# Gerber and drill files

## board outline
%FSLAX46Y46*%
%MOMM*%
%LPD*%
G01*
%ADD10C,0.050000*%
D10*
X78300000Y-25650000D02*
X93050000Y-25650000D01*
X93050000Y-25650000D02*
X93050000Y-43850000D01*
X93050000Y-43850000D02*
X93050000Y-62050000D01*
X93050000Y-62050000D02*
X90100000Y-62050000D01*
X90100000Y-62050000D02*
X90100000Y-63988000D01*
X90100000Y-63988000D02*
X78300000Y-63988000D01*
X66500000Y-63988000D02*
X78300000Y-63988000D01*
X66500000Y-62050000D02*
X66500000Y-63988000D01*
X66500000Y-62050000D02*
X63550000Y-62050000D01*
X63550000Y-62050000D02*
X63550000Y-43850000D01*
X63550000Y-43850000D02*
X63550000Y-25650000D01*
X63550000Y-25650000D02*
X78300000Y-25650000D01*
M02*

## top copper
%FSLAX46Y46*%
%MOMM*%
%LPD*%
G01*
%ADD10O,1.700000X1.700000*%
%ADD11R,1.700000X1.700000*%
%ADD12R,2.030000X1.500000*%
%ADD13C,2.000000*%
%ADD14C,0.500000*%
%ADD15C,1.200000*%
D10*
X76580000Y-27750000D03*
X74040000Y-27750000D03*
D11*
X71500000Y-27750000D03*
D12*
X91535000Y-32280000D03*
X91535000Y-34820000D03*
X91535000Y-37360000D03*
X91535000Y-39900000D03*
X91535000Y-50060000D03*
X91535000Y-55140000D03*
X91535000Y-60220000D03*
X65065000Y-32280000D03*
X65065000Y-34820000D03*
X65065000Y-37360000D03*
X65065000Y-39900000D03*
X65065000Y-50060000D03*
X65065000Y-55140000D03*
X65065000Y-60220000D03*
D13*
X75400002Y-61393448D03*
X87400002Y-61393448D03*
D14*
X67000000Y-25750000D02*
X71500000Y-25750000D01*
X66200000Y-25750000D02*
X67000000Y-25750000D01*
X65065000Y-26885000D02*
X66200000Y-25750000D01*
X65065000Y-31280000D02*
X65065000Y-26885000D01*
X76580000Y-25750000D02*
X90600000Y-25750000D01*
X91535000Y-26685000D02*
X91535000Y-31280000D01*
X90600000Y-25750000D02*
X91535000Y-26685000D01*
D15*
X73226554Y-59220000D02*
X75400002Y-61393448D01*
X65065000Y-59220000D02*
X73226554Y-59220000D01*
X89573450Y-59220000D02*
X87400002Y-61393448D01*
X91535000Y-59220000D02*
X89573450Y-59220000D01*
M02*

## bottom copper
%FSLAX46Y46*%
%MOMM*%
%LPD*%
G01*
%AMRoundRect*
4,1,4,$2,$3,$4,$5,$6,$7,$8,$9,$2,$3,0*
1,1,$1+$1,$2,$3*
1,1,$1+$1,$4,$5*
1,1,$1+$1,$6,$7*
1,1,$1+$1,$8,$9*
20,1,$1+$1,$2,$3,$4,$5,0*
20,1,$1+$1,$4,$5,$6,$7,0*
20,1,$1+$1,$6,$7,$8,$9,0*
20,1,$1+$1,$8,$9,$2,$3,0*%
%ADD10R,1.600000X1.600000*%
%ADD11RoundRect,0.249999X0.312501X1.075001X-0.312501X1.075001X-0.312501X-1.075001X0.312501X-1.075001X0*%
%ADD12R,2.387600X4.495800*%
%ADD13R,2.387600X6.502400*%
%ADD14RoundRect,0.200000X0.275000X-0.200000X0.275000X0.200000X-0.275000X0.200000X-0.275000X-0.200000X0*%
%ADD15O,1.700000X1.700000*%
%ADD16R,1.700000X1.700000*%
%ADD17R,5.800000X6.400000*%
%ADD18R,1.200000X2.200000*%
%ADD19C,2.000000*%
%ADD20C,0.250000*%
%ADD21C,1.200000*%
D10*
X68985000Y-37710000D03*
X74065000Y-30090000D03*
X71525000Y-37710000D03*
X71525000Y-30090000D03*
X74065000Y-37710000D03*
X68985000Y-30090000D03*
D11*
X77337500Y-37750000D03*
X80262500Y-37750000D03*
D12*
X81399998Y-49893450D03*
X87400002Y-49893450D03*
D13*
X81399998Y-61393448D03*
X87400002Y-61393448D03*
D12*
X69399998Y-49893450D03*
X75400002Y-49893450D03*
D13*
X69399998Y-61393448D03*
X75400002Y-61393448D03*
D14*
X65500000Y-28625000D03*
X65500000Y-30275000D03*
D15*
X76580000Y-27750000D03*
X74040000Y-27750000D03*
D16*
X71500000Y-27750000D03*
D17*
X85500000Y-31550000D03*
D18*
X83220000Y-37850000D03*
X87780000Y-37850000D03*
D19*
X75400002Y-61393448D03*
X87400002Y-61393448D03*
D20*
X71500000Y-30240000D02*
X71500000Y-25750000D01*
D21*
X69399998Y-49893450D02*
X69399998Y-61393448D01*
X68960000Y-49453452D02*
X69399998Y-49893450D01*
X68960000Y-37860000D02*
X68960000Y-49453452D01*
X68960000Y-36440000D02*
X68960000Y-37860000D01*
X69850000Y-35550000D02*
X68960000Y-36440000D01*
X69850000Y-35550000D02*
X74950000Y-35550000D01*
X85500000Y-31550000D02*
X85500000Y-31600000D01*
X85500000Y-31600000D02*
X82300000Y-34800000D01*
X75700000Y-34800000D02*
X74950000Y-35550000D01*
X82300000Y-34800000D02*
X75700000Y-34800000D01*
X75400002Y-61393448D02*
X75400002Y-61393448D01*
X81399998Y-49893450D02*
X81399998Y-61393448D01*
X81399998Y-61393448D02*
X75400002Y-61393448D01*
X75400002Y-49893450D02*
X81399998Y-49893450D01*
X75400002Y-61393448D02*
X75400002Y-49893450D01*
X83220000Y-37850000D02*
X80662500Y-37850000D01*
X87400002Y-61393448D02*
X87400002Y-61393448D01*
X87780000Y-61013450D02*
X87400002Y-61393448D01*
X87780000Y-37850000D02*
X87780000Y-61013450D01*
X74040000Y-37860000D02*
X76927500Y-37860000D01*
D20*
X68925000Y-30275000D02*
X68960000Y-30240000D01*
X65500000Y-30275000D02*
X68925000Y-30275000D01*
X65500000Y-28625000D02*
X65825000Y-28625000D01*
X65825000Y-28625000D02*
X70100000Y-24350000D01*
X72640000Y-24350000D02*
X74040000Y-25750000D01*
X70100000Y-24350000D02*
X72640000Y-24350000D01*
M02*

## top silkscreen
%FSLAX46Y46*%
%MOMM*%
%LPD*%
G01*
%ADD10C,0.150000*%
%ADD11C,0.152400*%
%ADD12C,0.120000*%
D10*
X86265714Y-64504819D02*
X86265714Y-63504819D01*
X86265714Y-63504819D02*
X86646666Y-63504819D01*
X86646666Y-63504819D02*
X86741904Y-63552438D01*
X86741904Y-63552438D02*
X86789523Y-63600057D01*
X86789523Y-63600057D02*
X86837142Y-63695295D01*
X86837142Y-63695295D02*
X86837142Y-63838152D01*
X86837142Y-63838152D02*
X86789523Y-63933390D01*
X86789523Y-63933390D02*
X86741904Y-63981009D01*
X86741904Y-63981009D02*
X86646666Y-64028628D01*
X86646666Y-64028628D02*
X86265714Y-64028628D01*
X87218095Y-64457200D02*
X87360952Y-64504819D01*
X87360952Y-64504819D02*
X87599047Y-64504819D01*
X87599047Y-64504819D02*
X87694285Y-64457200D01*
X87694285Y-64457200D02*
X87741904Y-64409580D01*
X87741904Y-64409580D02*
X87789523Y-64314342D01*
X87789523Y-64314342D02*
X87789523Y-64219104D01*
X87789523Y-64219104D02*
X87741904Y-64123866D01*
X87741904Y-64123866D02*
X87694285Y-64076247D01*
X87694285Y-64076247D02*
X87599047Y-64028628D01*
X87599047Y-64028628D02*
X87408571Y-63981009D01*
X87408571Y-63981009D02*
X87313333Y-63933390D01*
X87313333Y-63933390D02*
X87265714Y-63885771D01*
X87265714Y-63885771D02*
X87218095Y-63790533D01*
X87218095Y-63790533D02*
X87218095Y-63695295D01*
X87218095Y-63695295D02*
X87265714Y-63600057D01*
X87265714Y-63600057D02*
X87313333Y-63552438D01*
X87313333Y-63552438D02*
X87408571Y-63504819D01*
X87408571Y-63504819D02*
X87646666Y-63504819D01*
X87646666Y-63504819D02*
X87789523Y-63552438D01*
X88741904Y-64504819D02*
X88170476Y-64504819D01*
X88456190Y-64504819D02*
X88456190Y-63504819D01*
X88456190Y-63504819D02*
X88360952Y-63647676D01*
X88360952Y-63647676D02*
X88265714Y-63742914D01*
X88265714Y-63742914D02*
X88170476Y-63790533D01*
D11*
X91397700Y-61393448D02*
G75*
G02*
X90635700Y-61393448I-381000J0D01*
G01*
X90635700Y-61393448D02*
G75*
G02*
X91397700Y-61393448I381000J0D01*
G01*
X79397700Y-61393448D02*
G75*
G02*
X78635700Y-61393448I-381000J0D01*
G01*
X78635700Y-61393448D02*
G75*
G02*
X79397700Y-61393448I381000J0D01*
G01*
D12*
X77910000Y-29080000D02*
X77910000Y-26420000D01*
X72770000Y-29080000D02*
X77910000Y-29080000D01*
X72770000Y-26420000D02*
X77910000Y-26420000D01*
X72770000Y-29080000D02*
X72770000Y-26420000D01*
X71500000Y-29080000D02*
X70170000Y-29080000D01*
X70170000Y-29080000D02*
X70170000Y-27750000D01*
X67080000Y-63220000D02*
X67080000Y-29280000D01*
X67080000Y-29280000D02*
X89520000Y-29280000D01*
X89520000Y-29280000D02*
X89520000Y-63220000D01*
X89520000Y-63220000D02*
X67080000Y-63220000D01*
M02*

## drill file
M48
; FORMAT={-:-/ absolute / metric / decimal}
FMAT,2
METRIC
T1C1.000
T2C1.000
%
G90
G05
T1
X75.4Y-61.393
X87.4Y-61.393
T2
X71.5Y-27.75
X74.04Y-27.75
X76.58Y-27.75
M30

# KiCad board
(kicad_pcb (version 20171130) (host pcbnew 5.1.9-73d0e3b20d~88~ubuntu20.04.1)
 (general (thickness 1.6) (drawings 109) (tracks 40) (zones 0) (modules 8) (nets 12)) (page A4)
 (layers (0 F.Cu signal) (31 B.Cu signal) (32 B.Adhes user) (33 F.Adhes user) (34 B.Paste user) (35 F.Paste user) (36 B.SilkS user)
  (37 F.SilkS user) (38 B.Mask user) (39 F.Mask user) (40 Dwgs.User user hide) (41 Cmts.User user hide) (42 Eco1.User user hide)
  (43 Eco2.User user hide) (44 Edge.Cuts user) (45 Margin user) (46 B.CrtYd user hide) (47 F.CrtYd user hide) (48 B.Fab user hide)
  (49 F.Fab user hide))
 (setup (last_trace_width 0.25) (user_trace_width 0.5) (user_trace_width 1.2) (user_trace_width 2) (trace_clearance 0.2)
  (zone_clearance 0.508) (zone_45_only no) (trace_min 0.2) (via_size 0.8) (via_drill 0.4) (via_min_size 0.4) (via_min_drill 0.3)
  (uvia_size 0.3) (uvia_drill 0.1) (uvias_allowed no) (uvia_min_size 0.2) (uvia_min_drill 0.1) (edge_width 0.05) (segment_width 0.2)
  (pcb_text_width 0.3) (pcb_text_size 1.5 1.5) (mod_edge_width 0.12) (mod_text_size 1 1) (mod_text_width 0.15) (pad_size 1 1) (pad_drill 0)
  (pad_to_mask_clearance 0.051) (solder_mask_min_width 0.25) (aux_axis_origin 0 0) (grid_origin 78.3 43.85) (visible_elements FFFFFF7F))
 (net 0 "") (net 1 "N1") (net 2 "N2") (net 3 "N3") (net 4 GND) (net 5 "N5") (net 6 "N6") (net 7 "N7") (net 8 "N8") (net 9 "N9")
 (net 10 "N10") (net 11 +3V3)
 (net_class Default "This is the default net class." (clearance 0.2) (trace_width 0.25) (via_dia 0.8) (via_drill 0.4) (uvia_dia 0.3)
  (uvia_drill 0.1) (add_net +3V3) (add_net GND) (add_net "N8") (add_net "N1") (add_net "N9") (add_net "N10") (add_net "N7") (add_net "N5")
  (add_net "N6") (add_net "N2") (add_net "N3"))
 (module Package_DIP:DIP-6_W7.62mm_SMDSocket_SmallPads (layer B.Cu) (at 71.525 33.9 270)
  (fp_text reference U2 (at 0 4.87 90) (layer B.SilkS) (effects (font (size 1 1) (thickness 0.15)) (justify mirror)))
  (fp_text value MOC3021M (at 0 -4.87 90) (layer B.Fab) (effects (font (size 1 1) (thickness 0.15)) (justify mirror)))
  (pad 6 smd rect (at 3.81 2.54 270) (size 1.6 1.6) (layers B.Cu B.Paste B.Mask) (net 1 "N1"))
  (pad 3 smd rect (at -3.81 -2.54 270) (size 1.6 1.6) (layers B.Cu B.Paste B.Mask) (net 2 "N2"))
  (pad 5 smd rect (at 3.81 0 270) (size 1.6 1.6) (layers B.Cu B.Paste B.Mask) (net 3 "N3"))
  (pad 2 smd rect (at -3.81 0 270) (size 1.6 1.6) (layers B.Cu B.Paste B.Mask) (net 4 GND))
  (pad 4 smd rect (at 3.81 -2.54 270) (size 1.6 1.6) (layers B.Cu B.Paste B.Mask) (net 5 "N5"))
  (pad 1 smd rect (at -3.81 2.54 270) (size 1.6 1.6) (layers B.Cu B.Paste B.Mask) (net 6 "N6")))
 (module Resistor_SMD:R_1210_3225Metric (layer B.Cu) (at 78.8 37.75 180)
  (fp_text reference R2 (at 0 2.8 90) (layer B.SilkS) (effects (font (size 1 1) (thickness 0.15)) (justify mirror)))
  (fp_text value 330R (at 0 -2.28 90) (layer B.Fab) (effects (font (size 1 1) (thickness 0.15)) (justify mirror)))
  (pad 2 smd roundrect (at 1.4625 0 180) (size 1.125 2.65) (layers B.Cu B.Paste B.Mask) (roundrect_rratio 0.2222213333333333) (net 5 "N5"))
  (pad 1 smd roundrect (at -1.4625 0 180) (size 1.125 2.65) (layers B.Cu B.Paste B.Mask) (roundrect_rratio 0.2222213333333333) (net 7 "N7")))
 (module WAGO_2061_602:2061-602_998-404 (layer B.Cu) (at 84.4 56.65 180)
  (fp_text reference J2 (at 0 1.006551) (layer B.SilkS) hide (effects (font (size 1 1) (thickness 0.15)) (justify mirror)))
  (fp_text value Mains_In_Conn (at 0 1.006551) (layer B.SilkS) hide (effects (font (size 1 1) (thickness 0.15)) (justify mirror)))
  (fp_circle (center -6.6167 -4.743448) (end -6.2357 -4.743448) (layer F.SilkS) (width 0.1524))
  (pad 2 smd rect (at 3.000002 6.75655 180) (size 2.3876 4.4958) (layers B.Cu B.Paste B.Mask) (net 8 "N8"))
  (pad 1 smd rect (at -3.000002 6.75655 180) (size 2.3876 4.4958) (layers B.Cu B.Paste B.Mask) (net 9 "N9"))
  (pad 2 smd rect (at 3.000002 -4.743448 180) (size 2.3876 6.5024) (layers B.Cu B.Paste B.Mask) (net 8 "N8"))
  (pad 1 smd rect (at -3.000002 -4.743448 180) (size 2.3876 6.5024) (layers B.Cu B.Paste B.Mask) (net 9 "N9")))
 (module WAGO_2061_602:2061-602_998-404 (layer B.Cu) (at 72.4 56.65 180)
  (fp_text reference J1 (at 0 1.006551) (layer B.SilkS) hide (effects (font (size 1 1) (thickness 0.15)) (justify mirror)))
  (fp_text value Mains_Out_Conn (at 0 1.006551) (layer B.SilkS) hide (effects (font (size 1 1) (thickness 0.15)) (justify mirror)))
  (fp_circle (center -6.6167 -4.743448) (end -6.2357 -4.743448) (layer F.SilkS) (width 0.1524))
  (pad 2 smd rect (at 3.000002 6.75655 180) (size 2.3876 4.4958) (layers B.Cu B.Paste B.Mask) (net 1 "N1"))
  (pad 1 smd rect (at -3.000002 6.75655 180) (size 2.3876 4.4958) (layers B.Cu B.Paste B.Mask) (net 8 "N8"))
  (pad 2 smd rect (at 3.000002 -4.743448 180) (size 2.3876 6.5024) (layers B.Cu B.Paste B.Mask) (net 1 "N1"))
  (pad 1 smd rect (at -3.000002 -4.743448 180) (size 2.3876 6.5024) (layers B.Cu B.Paste B.Mask) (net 8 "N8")))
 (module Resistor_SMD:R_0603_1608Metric (layer B.Cu) (at 65.5 29.45 90)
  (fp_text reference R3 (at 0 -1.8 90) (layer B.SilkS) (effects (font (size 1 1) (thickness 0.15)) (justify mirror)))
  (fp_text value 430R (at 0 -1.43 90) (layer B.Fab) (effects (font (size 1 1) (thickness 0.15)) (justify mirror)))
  (pad 2 smd roundrect (at 0.825 0 90) (size 0.8 0.95) (layers B.Cu B.Paste B.Mask) (roundrect_rratio 0.25) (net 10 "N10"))
  (pad 1 smd roundrect (at -0.825 0 90) (size 0.8 0.95) (layers B.Cu B.Paste B.Mask) (roundrect_rratio 0.25) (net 6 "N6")))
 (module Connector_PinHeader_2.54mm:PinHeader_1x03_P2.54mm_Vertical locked (layer F.Cu) (at 71.500 27.750 90.000)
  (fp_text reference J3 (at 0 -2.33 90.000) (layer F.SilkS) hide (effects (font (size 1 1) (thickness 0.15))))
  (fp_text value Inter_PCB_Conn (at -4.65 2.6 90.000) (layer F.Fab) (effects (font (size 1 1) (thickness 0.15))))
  (fp_line (start -1.33 6.41) (end 1.33 6.41) (layer F.SilkS) (width 0.12))
  (fp_line (start -1.33 1.27) (end -1.33 6.41) (layer F.SilkS) (width 0.12))
  (fp_line (start 1.33 1.27) (end 1.33 6.41) (layer F.SilkS) (width 0.12))
  (fp_line (start -1.33 1.27) (end 1.33 1.27) (layer F.SilkS) (width 0.12))
  (fp_line (start -1.33 0) (end -1.33 -1.33) (layer F.SilkS) (width 0.12))
  (fp_line (start -1.33 -1.33) (end 0 -1.33) (layer F.SilkS) (width 0.12))
  (pad 3 thru_hole oval (at 0 5.08 90.000) (size 1.7 1.7) (drill 1) (layers *.Cu *.Mask) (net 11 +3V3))
  (pad 2 thru_hole oval (at 0 2.54 90.000) (size 1.7 1.7) (drill 1) (layers *.Cu *.Mask) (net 10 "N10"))
  (pad 1 thru_hole rect (at 0 0 90.000) (size 1.7 1.7) (drill 1) (layers *.Cu *.Mask) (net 4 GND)))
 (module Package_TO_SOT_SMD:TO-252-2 (layer B.Cu) (at 85.5 33.65 90)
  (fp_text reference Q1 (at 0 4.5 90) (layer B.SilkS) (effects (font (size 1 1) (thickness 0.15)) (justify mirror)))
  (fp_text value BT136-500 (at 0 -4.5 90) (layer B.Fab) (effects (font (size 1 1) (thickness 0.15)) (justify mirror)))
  (pad "" smd rect (at 0.425 -1.525 90) (size 3.05 2.75) (layers B.Paste))
  (pad "" smd rect (at 3.775 1.525 90) (size 3.05 2.75) (layers B.Paste))
  (pad "" smd rect (at 0.425 1.525 90) (size 3.05 2.75) (layers B.Paste))
  (pad "" smd rect (at 3.775 -1.525 90) (size 3.05 2.75) (layers B.Paste))
  (pad 2 smd rect (at 2.1 0 90) (size 6.4 5.8) (layers B.Cu B.Mask) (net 1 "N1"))
  (pad 3 smd rect (at -4.2 -2.28 90) (size 2.2 1.2) (layers B.Cu B.Paste B.Mask) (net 7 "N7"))
  (pad 1 smd rect (at -4.2 2.28 90) (size 2.2 1.2) (layers B.Cu B.Paste B.Mask) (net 9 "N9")))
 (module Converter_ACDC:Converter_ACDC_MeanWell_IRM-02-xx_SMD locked (layer F.Cu) (at 78.300 46.250 180.000)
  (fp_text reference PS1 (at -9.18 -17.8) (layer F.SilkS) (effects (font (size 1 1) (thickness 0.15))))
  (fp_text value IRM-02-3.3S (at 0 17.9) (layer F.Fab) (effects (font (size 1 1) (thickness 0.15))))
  (fp_line (start 11.22 -16.97) (end 11.22 16.97) (layer F.SilkS) (width 0.12))
  (fp_line (start 11.22 16.97) (end -11.22 16.97) (layer F.SilkS) (width 0.12))
  (fp_line (start -11.22 16.97) (end -11.22 -16.97) (layer F.SilkS) (width 0.12))
  (fp_line (start -11.22 -16.97) (end 11.22 -16.97) (layer F.SilkS) (width 0.12))
  (pad 12 smd rect (at -13.235 13.97 90.000) (size 1.5 2.03) (layers F.Cu F.Paste F.Mask) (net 11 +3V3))
  (pad 11 smd rect (at -13.235 11.43 90.000) (size 1.5 2.03) (layers F.Cu F.Paste F.Mask))
  (pad 10 smd rect (at -13.235 8.89 90.000) (size 1.5 2.03) (layers F.Cu F.Paste F.Mask))
  (pad 9 smd rect (at -13.235 6.35 90.000) (size 1.5 2.03) (layers F.Cu F.Paste F.Mask))
  (pad 5 smd rect (at -13.235 -3.81 90.000) (size 1.5 2.03) (layers F.Cu F.Paste F.Mask))
  (pad 3 smd rect (at -13.235 -8.89 90.000) (size 1.5 2.03) (layers F.Cu F.Paste F.Mask))
  (pad 1 smd rect (at -13.235 -13.97 90.000) (size 1.5 2.03) (layers F.Cu F.Paste F.Mask) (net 9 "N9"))
  (pad 13 smd rect (at 13.235 13.97 90.000) (size 1.5 2.03) (layers F.Cu F.Paste F.Mask) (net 4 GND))
  (pad 14 smd rect (at 13.235 11.43 90.000) (size 1.5 2.03) (layers F.Cu F.Paste F.Mask))
  (pad 15 smd rect (at 13.235 8.89 90.000) (size 1.5 2.03) (layers F.Cu F.Paste F.Mask))
  (pad 16 smd rect (at 13.235 6.35 90.000) (size 1.5 2.03) (layers F.Cu F.Paste F.Mask))
  (pad 20 smd rect (at 13.235 -3.81 90.000) (size 1.5 2.03) (layers F.Cu F.Paste F.Mask))
  (pad 22 smd rect (at 13.235 -8.89 90.000) (size 1.5 2.03) (layers F.Cu F.Paste F.Mask))
  (pad 24 smd rect (at 13.235 -13.97 90.000) (size 1.5 2.03) (layers F.Cu F.Paste F.Mask) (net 8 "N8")))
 (segment (start 71.5 30.24) (end 71.5 25.75) (width 0.25) (layer B.Cu) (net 4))
 (segment (start 67 25.75) (end 71.5 25.75) (width 0.5) (layer F.Cu) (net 4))
 (segment (start 66.2 25.75) (end 67 25.75) (width 0.5) (layer F.Cu) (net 4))
 (segment (start 65.065 26.885) (end 66.2 25.75) (width 0.5) (layer F.Cu) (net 4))
 (segment (start 65.065 31.28) (end 65.065 26.885) (width 0.5) (layer F.Cu) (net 4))
 (segment (start 76.58 25.75) (end 90.6 25.75) (width 0.5) (layer F.Cu) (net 11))
 (segment (start 91.535 26.685) (end 91.535 31.28) (width 0.5) (layer F.Cu) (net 11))
 (segment (start 90.6 25.75) (end 91.535 26.685) (width 0.5) (layer F.Cu) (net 11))
 (segment (start 69.399998 49.89345) (end 69.399998 61.393448) (width 1.2) (layer B.Cu) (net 1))
 (segment (start 68.96 49.453452) (end 69.399998 49.89345) (width 1.2) (layer B.Cu) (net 1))
 (segment (start 68.96 37.86) (end 68.96 49.453452) (width 1.2) (layer B.Cu) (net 1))
 (segment (start 68.96 36.44) (end 68.96 37.86) (width 1.2) (layer B.Cu) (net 1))
 (segment (start 69.85 35.55) (end 68.96 36.44) (width 1.2) (layer B.Cu) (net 1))
 (segment (start 69.85 35.55) (end 74.95 35.55) (width 1.2) (layer B.Cu) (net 1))
 (segment (start 85.5 31.55) (end 85.5 31.6) (width 1.2) (layer B.Cu) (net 1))
 (segment (start 85.5 31.6) (end 82.3 34.8) (width 1.2) (layer B.Cu) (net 1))
 (segment (start 75.7 34.8) (end 74.95 35.55) (width 1.2) (layer B.Cu) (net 1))
 (segment (start 82.3 34.8) (end 75.7 34.8) (width 1.2) (layer B.Cu) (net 1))
 (segment (start 75.400002 61.393448) (end 75.400002 61.393448) (width 1.2) (layer B.Cu) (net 8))
 (segment (start 81.399998 49.89345) (end 81.399998 61.393448) (width 1.2) (layer B.Cu) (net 8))
 (segment (start 81.399998 61.393448) (end 75.400002 61.393448) (width 1.2) (layer B.Cu) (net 8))
 (segment (start 75.400002 49.89345) (end 81.399998 49.89345) (width 1.2) (layer B.Cu) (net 8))
 (segment (start 75.400002 61.393448) (end 75.400002 49.89345) (width 1.2) (layer B.Cu) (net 8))
 (via (at 75.400002 61.393448) (size 2) (drill 1) (layers F.Cu B.Cu) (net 8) (status 1000000))
 (segment (start 73.226554 59.22) (end 75.400002 61.393448) (width 1.2) (layer F.Cu) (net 8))
 (segment (start 65.065 59.22) (end 73.226554 59.22) (width 1.2) (layer F.Cu) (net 8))
 (segment (start 83.22 37.85) (end 80.6625 37.85) (width 1.2) (layer B.Cu) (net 7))
 (segment (start 87.400002 61.393448) (end 87.400002 61.393448) (width 1.2) (layer B.Cu) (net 9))
 (via (at 87.400002 61.393448) (size 2) (drill 1) (layers F.Cu B.Cu) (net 9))
 (segment (start 89.57345 59.22) (end 87.400002 61.393448) (width 1.2) (layer F.Cu) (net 9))
 (segment (start 91.535 59.22) (end 89.57345 59.22) (width 1.2) (layer F.Cu) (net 9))
 (segment (start 87.78 61.01345) (end 87.400002 61.393448) (width 1.2) (layer B.Cu) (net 9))
 (segment (start 87.78 37.85) (end 87.78 61.01345) (width 1.2) (layer B.Cu) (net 9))
 (segment (start 74.04 37.86) (end 76.9275 37.86) (width 1.2) (layer B.Cu) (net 5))
 (segment (start 68.925 30.275) (end 68.96 30.24) (width 0.25) (layer B.Cu) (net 6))
 (segment (start 65.5 30.275) (end 68.925 30.275) (width 0.25) (layer B.Cu) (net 6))
 (segment (start 65.5 28.625) (end 65.825 28.625) (width 0.25) (layer B.Cu) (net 10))
 (segment (start 65.825 28.625) (end 70.1 24.35) (width 0.25) (layer B.Cu) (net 10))
 (segment (start 72.64 24.35) (end 74.04 25.75) (width 0.25) (layer B.Cu) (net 10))
 (segment (start 70.1 24.35) (end 72.64 24.35) (width 0.25) (layer B.Cu) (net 10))
 (gr_line (start 78.300 25.650) (end 93.050 25.650) (angle 90) (layer Edge.Cuts) (width 0.05))
 (gr_line (start 93.050 25.650) (end 93.050 43.850) (angle 90) (layer Edge.Cuts) (width 0.05))
 (gr_line (start 93.050 43.850) (end 93.050 62.050) (angle 90) (layer Edge.Cuts) (width 0.05))
 (gr_line (start 93.050 62.050) (end 90.100 62.050) (angle 90) (layer Edge.Cuts) (width 0.05))
 (gr_line (start 90.100 62.050) (end 90.100 63.988) (angle 90) (layer Edge.Cuts) (width 0.05))
 (gr_line (start 90.100 63.988) (end 78.300 63.988) (angle 90) (layer Edge.Cuts) (width 0.05))
 (gr_line (start 66.500 63.988) (end 78.300 63.988) (angle 90) (layer Edge.Cuts) (width 0.05))
 (gr_line (start 66.500 62.050) (end 66.500 63.988) (angle 90) (layer Edge.Cuts) (width 0.05))
 (gr_line (start 66.500 62.050) (end 63.550 62.050) (angle 90) (layer Edge.Cuts) (width 0.05))
 (gr_line (start 63.550 62.050) (end 63.550 43.850) (angle 90) (layer Edge.Cuts) (width 0.05))
 (gr_line (start 63.550 43.850) (end 63.550 25.650) (angle 90) (layer Edge.Cuts) (width 0.05))
 (gr_line (start 63.550 25.650) (end 78.300 25.650) (angle 90) (layer Edge.Cuts) (width 0.05)))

